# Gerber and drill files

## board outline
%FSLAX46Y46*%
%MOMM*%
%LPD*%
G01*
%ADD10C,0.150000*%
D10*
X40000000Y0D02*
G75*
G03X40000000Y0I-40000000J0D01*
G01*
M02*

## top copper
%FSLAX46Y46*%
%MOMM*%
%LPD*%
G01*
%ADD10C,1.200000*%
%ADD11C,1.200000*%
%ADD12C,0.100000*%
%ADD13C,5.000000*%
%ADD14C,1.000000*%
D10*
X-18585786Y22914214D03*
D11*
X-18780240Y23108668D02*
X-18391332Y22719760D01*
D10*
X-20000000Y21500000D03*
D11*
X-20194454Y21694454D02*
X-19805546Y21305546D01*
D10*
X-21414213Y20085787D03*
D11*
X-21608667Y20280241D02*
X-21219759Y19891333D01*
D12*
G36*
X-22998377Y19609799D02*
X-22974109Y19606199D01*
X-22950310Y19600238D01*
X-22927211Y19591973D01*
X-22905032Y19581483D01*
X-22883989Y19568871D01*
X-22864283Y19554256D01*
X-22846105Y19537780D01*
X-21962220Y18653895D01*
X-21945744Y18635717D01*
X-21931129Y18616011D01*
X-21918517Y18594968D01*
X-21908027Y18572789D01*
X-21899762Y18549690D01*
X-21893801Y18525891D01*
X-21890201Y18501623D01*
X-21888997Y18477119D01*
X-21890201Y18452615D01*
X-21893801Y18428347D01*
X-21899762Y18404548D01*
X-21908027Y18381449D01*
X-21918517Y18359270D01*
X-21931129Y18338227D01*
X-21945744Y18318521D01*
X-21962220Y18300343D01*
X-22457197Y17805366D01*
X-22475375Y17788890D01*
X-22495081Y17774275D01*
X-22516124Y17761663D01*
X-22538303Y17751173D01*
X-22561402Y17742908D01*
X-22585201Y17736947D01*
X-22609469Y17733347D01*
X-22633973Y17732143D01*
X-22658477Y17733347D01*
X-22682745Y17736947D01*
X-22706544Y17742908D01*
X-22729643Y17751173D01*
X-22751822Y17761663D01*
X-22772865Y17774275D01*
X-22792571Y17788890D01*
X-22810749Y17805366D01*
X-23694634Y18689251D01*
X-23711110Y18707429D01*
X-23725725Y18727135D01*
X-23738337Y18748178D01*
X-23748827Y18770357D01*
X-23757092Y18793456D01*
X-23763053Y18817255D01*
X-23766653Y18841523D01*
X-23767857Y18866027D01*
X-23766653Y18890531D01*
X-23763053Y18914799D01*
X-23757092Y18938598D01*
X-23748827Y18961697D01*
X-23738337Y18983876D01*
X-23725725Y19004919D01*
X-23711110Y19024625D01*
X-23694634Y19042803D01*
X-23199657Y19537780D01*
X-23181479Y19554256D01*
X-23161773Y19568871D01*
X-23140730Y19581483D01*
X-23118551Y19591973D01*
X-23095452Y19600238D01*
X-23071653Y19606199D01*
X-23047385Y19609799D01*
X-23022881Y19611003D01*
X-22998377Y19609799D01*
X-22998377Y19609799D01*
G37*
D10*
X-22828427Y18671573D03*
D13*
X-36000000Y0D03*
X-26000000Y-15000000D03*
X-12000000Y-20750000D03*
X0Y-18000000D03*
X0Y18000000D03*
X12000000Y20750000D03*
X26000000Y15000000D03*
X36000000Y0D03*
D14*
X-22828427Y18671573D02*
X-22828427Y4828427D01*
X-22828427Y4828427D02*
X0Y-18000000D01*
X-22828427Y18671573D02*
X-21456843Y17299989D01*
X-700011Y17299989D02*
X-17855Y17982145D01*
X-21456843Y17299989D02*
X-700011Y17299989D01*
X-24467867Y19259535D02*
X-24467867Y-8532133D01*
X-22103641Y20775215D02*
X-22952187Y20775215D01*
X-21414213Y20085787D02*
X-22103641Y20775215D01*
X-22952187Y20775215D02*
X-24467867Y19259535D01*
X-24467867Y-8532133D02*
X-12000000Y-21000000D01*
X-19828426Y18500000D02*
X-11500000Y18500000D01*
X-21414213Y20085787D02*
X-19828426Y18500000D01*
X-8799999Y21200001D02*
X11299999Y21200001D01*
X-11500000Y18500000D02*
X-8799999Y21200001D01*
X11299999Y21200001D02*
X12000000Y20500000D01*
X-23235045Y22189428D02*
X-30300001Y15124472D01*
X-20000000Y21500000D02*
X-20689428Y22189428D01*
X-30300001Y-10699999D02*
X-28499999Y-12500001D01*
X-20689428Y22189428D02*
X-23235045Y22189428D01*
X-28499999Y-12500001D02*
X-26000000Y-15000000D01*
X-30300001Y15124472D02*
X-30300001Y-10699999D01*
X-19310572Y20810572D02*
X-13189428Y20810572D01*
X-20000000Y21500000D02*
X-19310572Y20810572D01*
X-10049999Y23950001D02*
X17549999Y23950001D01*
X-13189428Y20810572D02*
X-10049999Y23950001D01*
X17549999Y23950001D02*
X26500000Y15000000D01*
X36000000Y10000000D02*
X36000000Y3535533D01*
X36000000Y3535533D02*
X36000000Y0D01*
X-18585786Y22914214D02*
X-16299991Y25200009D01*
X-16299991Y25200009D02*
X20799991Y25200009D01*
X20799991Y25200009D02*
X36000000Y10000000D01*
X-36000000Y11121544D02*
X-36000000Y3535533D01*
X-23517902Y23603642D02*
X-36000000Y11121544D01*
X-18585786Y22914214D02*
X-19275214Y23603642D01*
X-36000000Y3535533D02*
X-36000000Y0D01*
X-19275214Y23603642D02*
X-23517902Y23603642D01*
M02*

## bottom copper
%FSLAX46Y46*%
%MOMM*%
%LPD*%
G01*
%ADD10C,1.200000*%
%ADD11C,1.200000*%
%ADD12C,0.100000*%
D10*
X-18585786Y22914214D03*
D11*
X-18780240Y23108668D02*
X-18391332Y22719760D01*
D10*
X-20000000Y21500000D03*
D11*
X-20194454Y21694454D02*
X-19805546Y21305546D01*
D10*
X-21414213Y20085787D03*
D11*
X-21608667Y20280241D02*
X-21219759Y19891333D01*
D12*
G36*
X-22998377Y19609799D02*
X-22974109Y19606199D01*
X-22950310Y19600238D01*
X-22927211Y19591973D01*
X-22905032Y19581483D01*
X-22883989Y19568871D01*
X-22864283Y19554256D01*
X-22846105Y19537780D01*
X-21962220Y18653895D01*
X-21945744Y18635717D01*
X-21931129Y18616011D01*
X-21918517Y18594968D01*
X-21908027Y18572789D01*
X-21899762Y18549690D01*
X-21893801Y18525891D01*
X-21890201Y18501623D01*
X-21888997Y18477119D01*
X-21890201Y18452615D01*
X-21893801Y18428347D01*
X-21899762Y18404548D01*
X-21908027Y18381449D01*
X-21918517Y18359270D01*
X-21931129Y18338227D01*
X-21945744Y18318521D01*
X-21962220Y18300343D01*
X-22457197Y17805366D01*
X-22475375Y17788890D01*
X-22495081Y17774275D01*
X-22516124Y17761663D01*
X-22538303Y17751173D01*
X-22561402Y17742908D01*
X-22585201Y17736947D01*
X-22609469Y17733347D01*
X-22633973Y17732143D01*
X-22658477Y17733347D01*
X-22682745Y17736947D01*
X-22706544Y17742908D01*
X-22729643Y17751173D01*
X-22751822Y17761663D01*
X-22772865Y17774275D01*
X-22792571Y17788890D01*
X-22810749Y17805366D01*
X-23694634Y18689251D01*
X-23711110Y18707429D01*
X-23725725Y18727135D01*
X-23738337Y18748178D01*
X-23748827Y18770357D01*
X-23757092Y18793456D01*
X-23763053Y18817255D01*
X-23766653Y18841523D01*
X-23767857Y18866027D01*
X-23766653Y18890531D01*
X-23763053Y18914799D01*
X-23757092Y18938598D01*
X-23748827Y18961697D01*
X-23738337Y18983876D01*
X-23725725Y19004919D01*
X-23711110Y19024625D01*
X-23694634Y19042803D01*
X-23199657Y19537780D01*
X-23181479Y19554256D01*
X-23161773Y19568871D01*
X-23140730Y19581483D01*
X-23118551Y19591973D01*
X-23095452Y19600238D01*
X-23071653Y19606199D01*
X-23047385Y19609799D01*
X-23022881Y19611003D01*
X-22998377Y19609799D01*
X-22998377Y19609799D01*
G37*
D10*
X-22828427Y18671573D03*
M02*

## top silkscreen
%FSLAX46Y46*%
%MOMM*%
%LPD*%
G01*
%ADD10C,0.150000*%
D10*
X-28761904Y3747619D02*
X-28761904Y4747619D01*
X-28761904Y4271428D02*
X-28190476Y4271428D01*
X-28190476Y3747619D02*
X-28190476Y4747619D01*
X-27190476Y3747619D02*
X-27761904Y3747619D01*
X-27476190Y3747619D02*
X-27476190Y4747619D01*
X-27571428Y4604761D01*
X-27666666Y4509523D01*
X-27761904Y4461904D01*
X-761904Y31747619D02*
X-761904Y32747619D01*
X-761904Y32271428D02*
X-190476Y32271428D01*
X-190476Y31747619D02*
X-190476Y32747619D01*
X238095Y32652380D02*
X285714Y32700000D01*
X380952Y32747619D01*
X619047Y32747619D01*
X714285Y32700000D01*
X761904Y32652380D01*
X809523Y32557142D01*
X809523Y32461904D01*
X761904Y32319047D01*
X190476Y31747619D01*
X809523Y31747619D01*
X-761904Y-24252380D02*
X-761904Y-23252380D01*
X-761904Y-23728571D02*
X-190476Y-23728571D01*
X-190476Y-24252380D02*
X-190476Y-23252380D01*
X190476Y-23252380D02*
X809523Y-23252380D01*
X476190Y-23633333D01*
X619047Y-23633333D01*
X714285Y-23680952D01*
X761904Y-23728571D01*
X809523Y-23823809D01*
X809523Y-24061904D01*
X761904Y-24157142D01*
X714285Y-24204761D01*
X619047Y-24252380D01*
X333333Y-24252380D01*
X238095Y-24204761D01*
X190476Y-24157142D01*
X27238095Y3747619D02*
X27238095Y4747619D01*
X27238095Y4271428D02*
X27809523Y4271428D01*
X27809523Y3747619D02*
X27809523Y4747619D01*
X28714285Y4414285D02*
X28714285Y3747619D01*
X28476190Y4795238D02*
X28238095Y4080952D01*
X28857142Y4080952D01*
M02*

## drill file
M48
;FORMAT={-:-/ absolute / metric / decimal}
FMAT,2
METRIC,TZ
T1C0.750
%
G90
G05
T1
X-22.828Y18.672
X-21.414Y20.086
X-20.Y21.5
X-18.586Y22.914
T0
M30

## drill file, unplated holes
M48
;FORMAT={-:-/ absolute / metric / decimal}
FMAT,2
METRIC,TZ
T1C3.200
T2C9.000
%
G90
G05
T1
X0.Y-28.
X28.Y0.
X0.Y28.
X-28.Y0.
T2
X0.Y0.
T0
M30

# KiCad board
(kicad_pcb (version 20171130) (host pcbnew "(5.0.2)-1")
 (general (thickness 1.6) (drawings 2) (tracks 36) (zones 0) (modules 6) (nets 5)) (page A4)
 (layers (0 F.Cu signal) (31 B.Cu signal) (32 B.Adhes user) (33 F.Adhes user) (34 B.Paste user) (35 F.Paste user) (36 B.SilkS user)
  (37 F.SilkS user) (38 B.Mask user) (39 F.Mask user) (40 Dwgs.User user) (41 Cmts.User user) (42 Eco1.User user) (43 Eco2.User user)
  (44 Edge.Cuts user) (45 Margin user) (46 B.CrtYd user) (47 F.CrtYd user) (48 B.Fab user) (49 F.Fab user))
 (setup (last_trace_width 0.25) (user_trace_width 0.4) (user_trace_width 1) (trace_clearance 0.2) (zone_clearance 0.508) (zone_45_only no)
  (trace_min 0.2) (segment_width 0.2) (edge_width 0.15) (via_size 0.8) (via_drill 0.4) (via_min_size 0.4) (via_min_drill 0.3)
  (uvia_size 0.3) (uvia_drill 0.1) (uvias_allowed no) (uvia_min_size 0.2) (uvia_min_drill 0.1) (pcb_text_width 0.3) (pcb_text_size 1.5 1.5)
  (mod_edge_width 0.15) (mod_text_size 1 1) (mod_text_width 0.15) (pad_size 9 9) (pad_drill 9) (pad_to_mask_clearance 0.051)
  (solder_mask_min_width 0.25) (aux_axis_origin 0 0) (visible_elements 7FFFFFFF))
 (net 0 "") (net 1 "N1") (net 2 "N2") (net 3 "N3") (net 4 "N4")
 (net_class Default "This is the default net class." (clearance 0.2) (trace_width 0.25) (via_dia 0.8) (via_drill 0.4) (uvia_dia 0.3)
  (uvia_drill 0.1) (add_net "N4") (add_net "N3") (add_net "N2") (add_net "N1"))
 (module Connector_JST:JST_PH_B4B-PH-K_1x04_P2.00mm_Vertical (layer B.Cu) (at -22.828427 -18.671573 45)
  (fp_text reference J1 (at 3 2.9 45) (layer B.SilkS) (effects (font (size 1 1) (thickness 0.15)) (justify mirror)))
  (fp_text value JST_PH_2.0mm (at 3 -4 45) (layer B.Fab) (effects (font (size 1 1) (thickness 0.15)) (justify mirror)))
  (pad 4 thru_hole oval (at 6 0 45) (size 1.2 1.75) (drill 0.75) (layers *.Cu *.Mask) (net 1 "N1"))
  (pad 3 thru_hole oval (at 4 0 45) (size 1.2 1.75) (drill 0.75) (layers *.Cu *.Mask) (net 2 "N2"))
  (pad 2 thru_hole oval (at 2.000001 0 45) (size 1.2 1.75) (drill 0.75) (layers *.Cu *.Mask) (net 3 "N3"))
  (pad 1 thru_hole roundrect (at 0 0 45) (size 1.2 1.75) (drill 0.75) (layers *.Cu *.Mask) (roundrect_rratio 0.208333) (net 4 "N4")))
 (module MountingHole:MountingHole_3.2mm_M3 (layer F.Cu) (at -28 0)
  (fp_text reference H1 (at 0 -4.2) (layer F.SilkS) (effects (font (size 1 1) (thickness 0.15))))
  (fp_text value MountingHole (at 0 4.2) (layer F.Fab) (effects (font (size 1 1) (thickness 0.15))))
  (pad 1 np_thru_hole circle (at 0 0) (size 3.2 3.2) (drill 3.2) (layers *.Cu *.Mask)))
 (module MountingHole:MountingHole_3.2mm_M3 (layer F.Cu) (at 0 -28)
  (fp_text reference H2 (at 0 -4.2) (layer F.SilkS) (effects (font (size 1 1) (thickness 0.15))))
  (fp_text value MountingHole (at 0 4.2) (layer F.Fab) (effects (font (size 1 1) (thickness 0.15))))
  (pad 1 np_thru_hole circle (at 0 0) (size 3.2 3.2) (drill 3.2) (layers *.Cu *.Mask)))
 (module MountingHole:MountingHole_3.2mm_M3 (layer F.Cu) (at 0 28)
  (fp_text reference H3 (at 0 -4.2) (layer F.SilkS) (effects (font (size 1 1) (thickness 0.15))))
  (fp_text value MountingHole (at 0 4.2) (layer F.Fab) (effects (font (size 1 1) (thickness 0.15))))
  (pad 1 np_thru_hole circle (at 0 0) (size 3.2 3.2) (drill 3.2) (layers *.Cu *.Mask)))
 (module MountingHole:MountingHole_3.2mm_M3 (layer F.Cu) (at 28 0)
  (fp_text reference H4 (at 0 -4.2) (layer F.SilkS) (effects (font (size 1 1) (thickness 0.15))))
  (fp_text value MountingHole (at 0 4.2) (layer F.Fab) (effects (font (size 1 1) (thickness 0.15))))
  (pad 1 np_thru_hole circle (at 0 0) (size 3.2 3.2) (drill 3.2) (layers *.Cu *.Mask)))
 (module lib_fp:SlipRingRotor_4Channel (layer F.Cu) (at 0 0)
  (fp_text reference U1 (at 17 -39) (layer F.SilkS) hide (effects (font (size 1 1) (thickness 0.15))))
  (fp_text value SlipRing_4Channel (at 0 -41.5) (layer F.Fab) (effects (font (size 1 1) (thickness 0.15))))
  (pad "" np_thru_hole circle (at 0 0) (size 9 9) (drill 9) (layers *.Cu *.Mask))
  (pad 4 smd circle (at -36 0) (size 5 5) (layers F.Cu F.Paste F.Mask) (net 1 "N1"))
  (pad 3 smd circle (at -26 15) (size 5 5) (layers F.Cu F.Paste F.Mask) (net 2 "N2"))
  (pad 2 smd circle (at -12 20.75) (size 5 5) (layers F.Cu F.Paste F.Mask) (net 3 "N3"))
  (pad 1 smd circle (at 0 18) (size 5 5) (layers F.Cu F.Paste F.Mask) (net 4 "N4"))
  (pad 1 smd circle (at 0 -18) (size 5 5) (layers F.Cu F.Paste F.Mask) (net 4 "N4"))
  (pad 2 smd circle (at 12 -20.75) (size 5 5) (layers F.Cu F.Paste F.Mask) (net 3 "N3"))
  (pad 3 smd circle (at 26 -15) (size 5 5) (layers F.Cu F.Paste F.Mask) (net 2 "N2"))
  (pad 4 smd circle (at 36 0) (size 5 5) (layers F.Cu F.Paste F.Mask) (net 1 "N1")))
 (gr_circle (center 0 0) (end 40 0) (layer Edge.Cuts) (width 0.15))
 (segment (start -22.828427 -18.671573) (end -22.828427 -4.828427) (width 1) (layer F.Cu) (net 4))
 (segment (start -22.828427 -4.828427) (end 0 18) (width 1) (layer F.Cu) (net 4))
 (segment (start -22.828427 -18.671573) (end -21.456843 -17.299989) (width 1) (layer F.Cu) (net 4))
 (segment (start -0.700011 -17.299989) (end -0.017855 -17.982145) (width 1) (layer F.Cu) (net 4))
 (segment (start -21.456843 -17.299989) (end -0.700011 -17.299989) (width 1) (layer F.Cu) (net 4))
 (segment (start -24.467867 -19.259535) (end -24.467867 8.532133) (width 1) (layer F.Cu) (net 3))
 (segment (start -22.103641 -20.775215) (end -22.952187 -20.775215) (width 1) (layer F.Cu) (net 3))
 (segment (start -21.414213 -20.085787) (end -22.103641 -20.775215) (width 1) (layer F.Cu) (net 3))
 (segment (start -22.952187 -20.775215) (end -24.467867 -19.259535) (width 1) (layer F.Cu) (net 3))
 (segment (start -24.467867 8.532133) (end -12 21) (width 1) (layer F.Cu) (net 3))
 (segment (start -19.828426 -18.5) (end -11.5 -18.5) (width 1) (layer F.Cu) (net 3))
 (segment (start -21.414213 -20.085787) (end -19.828426 -18.5) (width 1) (layer F.Cu) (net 3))
 (segment (start -8.799999 -21.200001) (end 11.299999 -21.200001) (width 1) (layer F.Cu) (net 3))
 (segment (start -11.5 -18.5) (end -8.799999 -21.200001) (width 1) (layer F.Cu) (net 3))
 (segment (start 11.299999 -21.200001) (end 12 -20.5) (width 1) (layer F.Cu) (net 3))
 (segment (start -23.235045 -22.189428) (end -30.300001 -15.124472) (width 1) (layer F.Cu) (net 2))
 (segment (start -20 -21.5) (end -20.689428 -22.189428) (width 1) (layer F.Cu) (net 2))
 (segment (start -30.300001 10.699999) (end -28.499999 12.500001) (width 1) (layer F.Cu) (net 2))
 (segment (start -20.689428 -22.189428) (end -23.235045 -22.189428) (width 1) (layer F.Cu) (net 2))
 (segment (start -28.499999 12.500001) (end -26 15) (width 1) (layer F.Cu) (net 2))
 (segment (start -30.300001 -15.124472) (end -30.300001 10.699999) (width 1) (layer F.Cu) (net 2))
 (segment (start -19.310572 -20.810572) (end -13.189428 -20.810572) (width 1) (layer F.Cu) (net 2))
 (segment (start -20 -21.5) (end -19.310572 -20.810572) (width 1) (layer F.Cu) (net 2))
 (segment (start -10.049999 -23.950001) (end 17.549999 -23.950001) (width 1) (layer F.Cu) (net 2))
 (segment (start -13.189428 -20.810572) (end -10.049999 -23.950001) (width 1) (layer F.Cu) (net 2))
 (segment (start 17.549999 -23.950001) (end 26.5 -15) (width 1) (layer F.Cu) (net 2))
 (segment (start 36 -10) (end 36 -3.535533) (width 1) (layer F.Cu) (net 1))
 (segment (start 36 -3.535533) (end 36 0) (width 1) (layer F.Cu) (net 1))
 (segment (start -18.585786 -22.914214) (end -16.299991 -25.200009) (width 1) (layer F.Cu) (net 1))
 (segment (start -16.299991 -25.200009) (end 20.799991 -25.200009) (width 1) (layer F.Cu) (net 1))
 (segment (start 20.799991 -25.200009) (end 36 -10) (width 1) (layer F.Cu) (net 1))
 (segment (start -36 -11.121544) (end -36 -3.535533) (width 1) (layer F.Cu) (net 1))
 (segment (start -23.517902 -23.603642) (end -36 -11.121544) (width 1) (layer F.Cu) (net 1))
 (segment (start -18.585786 -22.914214) (end -19.275214 -23.603642) (width 1) (layer F.Cu) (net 1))
 (segment (start -36 -3.535533) (end -36 0) (width 1) (layer F.Cu) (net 1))
 (segment (start -19.275214 -23.603642) (end -23.517902 -23.603642) (width 1) (layer F.Cu) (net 1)))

